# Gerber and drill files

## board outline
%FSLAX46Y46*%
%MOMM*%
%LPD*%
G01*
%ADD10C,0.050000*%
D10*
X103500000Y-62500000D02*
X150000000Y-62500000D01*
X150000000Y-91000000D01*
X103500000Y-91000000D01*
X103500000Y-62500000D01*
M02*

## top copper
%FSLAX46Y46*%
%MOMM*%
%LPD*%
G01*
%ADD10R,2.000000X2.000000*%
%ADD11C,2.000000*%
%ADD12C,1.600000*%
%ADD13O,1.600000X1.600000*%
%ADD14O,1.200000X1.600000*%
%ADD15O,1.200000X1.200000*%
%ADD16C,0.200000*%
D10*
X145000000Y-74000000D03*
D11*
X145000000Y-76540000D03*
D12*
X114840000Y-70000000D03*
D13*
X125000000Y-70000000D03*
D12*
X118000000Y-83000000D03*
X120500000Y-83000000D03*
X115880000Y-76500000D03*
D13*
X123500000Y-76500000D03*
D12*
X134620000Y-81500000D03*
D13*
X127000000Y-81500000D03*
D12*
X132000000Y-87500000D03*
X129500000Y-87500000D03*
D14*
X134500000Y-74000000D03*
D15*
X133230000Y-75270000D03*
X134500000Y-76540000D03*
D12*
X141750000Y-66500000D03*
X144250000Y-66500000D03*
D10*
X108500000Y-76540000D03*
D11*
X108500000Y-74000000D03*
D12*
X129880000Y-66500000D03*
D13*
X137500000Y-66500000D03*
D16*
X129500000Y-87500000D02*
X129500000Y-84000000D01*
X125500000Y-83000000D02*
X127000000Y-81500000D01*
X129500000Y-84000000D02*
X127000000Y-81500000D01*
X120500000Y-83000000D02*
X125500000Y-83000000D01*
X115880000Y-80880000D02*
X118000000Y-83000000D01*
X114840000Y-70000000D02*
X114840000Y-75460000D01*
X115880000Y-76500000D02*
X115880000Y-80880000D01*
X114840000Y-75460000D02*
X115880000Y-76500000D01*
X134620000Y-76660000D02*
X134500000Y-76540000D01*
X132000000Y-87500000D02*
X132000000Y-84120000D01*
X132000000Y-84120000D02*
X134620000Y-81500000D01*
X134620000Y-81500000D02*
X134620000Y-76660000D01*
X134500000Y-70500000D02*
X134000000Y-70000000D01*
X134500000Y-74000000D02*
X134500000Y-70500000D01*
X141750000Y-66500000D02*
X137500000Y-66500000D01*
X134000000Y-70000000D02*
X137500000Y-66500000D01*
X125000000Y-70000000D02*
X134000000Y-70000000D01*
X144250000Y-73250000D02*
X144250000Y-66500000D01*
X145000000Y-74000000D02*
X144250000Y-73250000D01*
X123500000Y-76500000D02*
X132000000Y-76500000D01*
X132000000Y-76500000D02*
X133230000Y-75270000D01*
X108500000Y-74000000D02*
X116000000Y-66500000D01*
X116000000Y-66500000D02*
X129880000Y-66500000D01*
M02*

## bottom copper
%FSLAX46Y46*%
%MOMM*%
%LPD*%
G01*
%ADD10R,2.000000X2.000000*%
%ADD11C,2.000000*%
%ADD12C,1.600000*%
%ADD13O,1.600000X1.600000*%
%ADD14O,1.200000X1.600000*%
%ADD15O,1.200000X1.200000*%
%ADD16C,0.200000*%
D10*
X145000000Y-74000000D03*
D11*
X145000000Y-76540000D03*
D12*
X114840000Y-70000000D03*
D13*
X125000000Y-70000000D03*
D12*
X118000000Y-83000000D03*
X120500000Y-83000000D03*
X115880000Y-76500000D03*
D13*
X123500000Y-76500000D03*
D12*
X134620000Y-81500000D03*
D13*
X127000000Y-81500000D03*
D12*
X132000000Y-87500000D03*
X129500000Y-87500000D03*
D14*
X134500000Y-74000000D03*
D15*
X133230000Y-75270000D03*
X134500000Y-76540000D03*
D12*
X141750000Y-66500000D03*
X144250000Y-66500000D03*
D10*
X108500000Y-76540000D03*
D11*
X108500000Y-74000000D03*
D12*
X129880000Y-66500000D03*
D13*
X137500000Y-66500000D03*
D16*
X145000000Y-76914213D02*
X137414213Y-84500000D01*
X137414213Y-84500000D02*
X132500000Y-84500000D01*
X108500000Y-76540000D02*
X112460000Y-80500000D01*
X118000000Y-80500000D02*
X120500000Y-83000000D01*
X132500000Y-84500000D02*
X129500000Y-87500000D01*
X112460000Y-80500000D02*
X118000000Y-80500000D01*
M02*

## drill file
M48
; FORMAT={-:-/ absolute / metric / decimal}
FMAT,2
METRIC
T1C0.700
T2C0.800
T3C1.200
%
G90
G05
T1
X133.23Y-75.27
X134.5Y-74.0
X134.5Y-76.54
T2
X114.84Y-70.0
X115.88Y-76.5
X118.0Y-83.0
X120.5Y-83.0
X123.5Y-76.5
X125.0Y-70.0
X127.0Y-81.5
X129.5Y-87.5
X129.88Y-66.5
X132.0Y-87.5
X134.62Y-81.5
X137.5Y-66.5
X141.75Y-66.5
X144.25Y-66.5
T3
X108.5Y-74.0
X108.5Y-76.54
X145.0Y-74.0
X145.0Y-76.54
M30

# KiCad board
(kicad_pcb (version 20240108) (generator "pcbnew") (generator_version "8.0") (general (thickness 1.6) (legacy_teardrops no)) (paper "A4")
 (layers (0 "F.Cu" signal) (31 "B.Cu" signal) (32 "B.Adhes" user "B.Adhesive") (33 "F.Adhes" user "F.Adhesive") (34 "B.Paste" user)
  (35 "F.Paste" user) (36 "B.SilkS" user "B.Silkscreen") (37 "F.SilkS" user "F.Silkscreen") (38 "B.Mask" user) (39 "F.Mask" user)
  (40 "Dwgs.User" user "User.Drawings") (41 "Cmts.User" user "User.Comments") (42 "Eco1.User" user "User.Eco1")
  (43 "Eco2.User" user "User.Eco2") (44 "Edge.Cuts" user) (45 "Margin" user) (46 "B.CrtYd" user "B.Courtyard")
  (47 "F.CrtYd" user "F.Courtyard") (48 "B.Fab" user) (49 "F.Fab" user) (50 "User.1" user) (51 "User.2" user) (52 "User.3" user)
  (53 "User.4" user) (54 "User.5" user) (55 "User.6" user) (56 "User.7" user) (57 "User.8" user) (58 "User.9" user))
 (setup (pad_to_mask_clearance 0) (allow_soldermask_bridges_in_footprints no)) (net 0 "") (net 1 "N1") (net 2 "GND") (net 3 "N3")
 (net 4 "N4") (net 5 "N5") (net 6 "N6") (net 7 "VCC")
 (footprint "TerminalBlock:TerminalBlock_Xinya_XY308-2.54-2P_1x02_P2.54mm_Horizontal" (layer "F.Cu") (at 145 74 -90)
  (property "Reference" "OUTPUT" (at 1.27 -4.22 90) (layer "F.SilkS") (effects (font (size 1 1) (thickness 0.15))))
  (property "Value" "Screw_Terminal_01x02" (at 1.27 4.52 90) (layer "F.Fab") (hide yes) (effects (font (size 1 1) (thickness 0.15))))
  (pad "1" thru_hole rect (at 0 0 270) (size 2 2) (drill 1.2) (layers "*.Cu" "*.Mask") (remove_unused_layers no) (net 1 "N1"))
  (pad "2" thru_hole circle (at 2.54 0 270) (size 2 2) (drill 1.2) (layers "*.Cu" "*.Mask") (remove_unused_layers no) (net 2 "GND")))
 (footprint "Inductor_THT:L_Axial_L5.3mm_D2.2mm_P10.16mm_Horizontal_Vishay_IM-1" (layer "F.Cu") (at 114.84 70)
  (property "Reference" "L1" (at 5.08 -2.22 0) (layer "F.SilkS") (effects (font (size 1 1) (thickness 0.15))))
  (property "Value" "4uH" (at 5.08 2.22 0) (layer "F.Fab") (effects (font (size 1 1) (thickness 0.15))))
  (pad "1" thru_hole circle (at 0 0) (size 1.6 1.6) (drill 0.8) (layers "*.Cu" "*.Mask") (remove_unused_layers no) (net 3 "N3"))
  (pad "2" thru_hole oval (at 10.16 0) (size 1.6 1.6) (drill 0.8) (layers "*.Cu" "*.Mask") (remove_unused_layers no) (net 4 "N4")))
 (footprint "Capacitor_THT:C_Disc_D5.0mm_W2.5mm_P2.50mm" (layer "F.Cu") (at 118 83)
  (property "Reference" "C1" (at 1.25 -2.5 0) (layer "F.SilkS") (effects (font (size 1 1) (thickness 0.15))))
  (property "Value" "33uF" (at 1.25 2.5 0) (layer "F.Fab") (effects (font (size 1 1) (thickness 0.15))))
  (pad "1" thru_hole circle (at 0 0) (size 1.6 1.6) (drill 0.8) (layers "*.Cu" "*.Mask") (remove_unused_layers no) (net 3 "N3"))
  (pad "2" thru_hole circle (at 2.5 0) (size 1.6 1.6) (drill 0.8) (layers "*.Cu" "*.Mask") (remove_unused_layers no) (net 2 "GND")))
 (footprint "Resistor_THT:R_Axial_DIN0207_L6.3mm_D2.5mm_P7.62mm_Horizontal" (layer "F.Cu") (at 115.88 76.5)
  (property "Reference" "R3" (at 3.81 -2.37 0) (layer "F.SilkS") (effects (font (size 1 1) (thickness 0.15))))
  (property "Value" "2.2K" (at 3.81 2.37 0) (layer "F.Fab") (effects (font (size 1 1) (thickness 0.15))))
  (pad "1" thru_hole circle (at 0 0) (size 1.6 1.6) (drill 0.8) (layers "*.Cu" "*.Mask") (remove_unused_layers no) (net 3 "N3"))
  (pad "2" thru_hole oval (at 7.62 0) (size 1.6 1.6) (drill 0.8) (layers "*.Cu" "*.Mask") (remove_unused_layers no) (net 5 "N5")))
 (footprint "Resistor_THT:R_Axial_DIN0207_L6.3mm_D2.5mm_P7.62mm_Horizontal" (layer "F.Cu") (at 134.62 81.5 180)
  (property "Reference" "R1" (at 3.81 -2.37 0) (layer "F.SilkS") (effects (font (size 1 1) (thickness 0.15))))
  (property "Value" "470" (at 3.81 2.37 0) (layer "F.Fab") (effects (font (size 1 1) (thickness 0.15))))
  (pad "1" thru_hole circle (at 0 0 180) (size 1.6 1.6) (drill 0.8) (layers "*.Cu" "*.Mask") (remove_unused_layers no) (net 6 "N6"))
  (pad "2" thru_hole oval (at 7.62 0 180) (size 1.6 1.6) (drill 0.8) (layers "*.Cu" "*.Mask") (remove_unused_layers no) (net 2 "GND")))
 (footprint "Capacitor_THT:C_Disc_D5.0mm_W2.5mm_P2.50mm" (layer "F.Cu") (at 132 87.5 180)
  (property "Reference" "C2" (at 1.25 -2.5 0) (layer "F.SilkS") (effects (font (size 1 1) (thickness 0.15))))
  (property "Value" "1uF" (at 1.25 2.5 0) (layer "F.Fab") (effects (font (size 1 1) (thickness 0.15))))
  (pad "1" thru_hole circle (at 0 0 180) (size 1.6 1.6) (drill 0.8) (layers "*.Cu" "*.Mask") (remove_unused_layers no) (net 6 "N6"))
  (pad "2" thru_hole circle (at 2.5 0 180) (size 1.6 1.6) (drill 0.8) (layers "*.Cu" "*.Mask") (remove_unused_layers no) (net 2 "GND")))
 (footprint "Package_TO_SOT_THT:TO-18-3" (layer "F.Cu") (at 134.5 74 -90)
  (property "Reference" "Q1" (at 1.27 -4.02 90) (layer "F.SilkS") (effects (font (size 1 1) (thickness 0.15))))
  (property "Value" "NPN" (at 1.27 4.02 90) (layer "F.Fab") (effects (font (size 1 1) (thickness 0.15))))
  (pad "1" thru_hole oval (at 0 0 270) (size 1.6 1.2) (drill 0.7) (layers "*.Cu" "*.Mask") (remove_unused_layers no) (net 4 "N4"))
  (pad "2" thru_hole oval (at 1.27 1.27 270) (size 1.2 1.2) (drill 0.7) (layers "*.Cu" "*.Mask") (remove_unused_layers no) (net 5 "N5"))
  (pad "3" thru_hole oval (at 2.54 0 270) (size 1.2 1.2) (drill 0.7) (layers "*.Cu" "*.Mask") (remove_unused_layers no) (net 6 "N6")))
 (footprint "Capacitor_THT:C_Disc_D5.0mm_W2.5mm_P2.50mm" (layer "F.Cu") (at 141.75 66.5)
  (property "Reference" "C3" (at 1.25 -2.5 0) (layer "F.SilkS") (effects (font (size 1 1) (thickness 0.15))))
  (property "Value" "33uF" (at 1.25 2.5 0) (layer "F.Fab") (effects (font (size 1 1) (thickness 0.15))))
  (pad "1" thru_hole circle (at 0 0) (size 1.6 1.6) (drill 0.8) (layers "*.Cu" "*.Mask") (remove_unused_layers no) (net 4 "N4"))
  (pad "2" thru_hole circle (at 2.5 0) (size 1.6 1.6) (drill 0.8) (layers "*.Cu" "*.Mask") (remove_unused_layers no) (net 1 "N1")))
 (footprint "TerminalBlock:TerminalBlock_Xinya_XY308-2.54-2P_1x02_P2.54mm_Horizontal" (layer "F.Cu") (at 108.5 76.54 90)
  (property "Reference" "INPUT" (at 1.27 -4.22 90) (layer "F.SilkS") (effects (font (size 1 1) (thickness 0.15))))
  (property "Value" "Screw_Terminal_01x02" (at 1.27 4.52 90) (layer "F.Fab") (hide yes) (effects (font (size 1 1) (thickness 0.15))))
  (pad "1" thru_hole rect (at 0 0 90) (size 2 2) (drill 1.2) (layers "*.Cu" "*.Mask") (remove_unused_layers no) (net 2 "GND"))
  (pad "2" thru_hole circle (at 2.54 0 90) (size 2 2) (drill 1.2) (layers "*.Cu" "*.Mask") (remove_unused_layers no) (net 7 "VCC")))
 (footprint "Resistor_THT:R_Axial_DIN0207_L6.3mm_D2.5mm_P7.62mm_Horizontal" (layer "F.Cu") (at 129.88 66.5)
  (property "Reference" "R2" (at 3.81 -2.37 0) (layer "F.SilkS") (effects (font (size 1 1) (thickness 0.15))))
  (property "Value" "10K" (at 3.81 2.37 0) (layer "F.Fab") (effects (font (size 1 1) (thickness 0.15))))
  (pad "1" thru_hole circle (at 0 0) (size 1.6 1.6) (drill 0.8) (layers "*.Cu" "*.Mask") (remove_unused_layers no) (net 7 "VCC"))
  (pad "2" thru_hole oval (at 7.62 0) (size 1.6 1.6) (drill 0.8) (layers "*.Cu" "*.Mask") (remove_unused_layers no) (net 4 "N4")))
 (gr_rect (start 103.5 62.5) (end 150 91) (stroke (width 0.05) (type default)) (fill none) (layer "Edge.Cuts"))
 (segment (start 129.5 87.5) (end 129.5 84) (width 0.2) (layer "F.Cu") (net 2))
 (segment (start 125.5 83) (end 127 81.5) (width 0.2) (layer "F.Cu") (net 2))
 (segment (start 129.5 84) (end 127 81.5) (width 0.2) (layer "F.Cu") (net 2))
 (segment (start 120.5 83) (end 125.5 83) (width 0.2) (layer "F.Cu") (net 2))
 (segment (start 145 76.914213) (end 137.414213 84.5) (width 0.2) (layer "B.Cu") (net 2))
 (segment (start 137.414213 84.5) (end 132.5 84.5) (width 0.2) (layer "B.Cu") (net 2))
 (segment (start 108.5 76.54) (end 112.46 80.5) (width 0.2) (layer "B.Cu") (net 2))
 (segment (start 118 80.5) (end 120.5 83) (width 0.2) (layer "B.Cu") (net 2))
 (segment (start 132.5 84.5) (end 129.5 87.5) (width 0.2) (layer "B.Cu") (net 2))
 (segment (start 112.46 80.5) (end 118 80.5) (width 0.2) (layer "B.Cu") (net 2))
 (segment (start 115.88 80.88) (end 118 83) (width 0.2) (layer "F.Cu") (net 3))
 (segment (start 114.84 70) (end 114.84 75.46) (width 0.2) (layer "F.Cu") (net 3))
 (segment (start 115.88 76.5) (end 115.88 80.88) (width 0.2) (layer "F.Cu") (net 3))
 (segment (start 114.84 75.46) (end 115.88 76.5) (width 0.2) (layer "F.Cu") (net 3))
 (segment (start 134.62 76.66) (end 134.5 76.54) (width 0.2) (layer "F.Cu") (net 6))
 (segment (start 132 87.5) (end 132 84.12) (width 0.2) (layer "F.Cu") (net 6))
 (segment (start 132 84.12) (end 134.62 81.5) (width 0.2) (layer "F.Cu") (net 6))
 (segment (start 134.62 81.5) (end 134.62 76.66) (width 0.2) (layer "F.Cu") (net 6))
 (segment (start 134.5 70.5) (end 134 70) (width 0.2) (layer "F.Cu") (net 4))
 (segment (start 134.5 74) (end 134.5 70.5) (width 0.2) (layer "F.Cu") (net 4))
 (segment (start 141.75 66.5) (end 137.5 66.5) (width 0.2) (layer "F.Cu") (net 4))
 (segment (start 134 70) (end 137.5 66.5) (width 0.2) (layer "F.Cu") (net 4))
 (segment (start 125 70) (end 134 70) (width 0.2) (layer "F.Cu") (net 4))
 (segment (start 144.25 73.25) (end 144.25 66.5) (width 0.2) (layer "F.Cu") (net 1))
 (segment (start 145 74) (end 144.25 73.25) (width 0.2) (layer "F.Cu") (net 1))
 (segment (start 123.5 76.5) (end 132 76.5) (width 0.2) (layer "F.Cu") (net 5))
 (segment (start 132 76.5) (end 133.23 75.27) (width 0.2) (layer "F.Cu") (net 5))
 (segment (start 108.5 74) (end 116 66.5) (width 0.2) (layer "F.Cu") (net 7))
 (segment (start 116 66.5) (end 129.88 66.5) (width 0.2) (layer "F.Cu") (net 7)))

